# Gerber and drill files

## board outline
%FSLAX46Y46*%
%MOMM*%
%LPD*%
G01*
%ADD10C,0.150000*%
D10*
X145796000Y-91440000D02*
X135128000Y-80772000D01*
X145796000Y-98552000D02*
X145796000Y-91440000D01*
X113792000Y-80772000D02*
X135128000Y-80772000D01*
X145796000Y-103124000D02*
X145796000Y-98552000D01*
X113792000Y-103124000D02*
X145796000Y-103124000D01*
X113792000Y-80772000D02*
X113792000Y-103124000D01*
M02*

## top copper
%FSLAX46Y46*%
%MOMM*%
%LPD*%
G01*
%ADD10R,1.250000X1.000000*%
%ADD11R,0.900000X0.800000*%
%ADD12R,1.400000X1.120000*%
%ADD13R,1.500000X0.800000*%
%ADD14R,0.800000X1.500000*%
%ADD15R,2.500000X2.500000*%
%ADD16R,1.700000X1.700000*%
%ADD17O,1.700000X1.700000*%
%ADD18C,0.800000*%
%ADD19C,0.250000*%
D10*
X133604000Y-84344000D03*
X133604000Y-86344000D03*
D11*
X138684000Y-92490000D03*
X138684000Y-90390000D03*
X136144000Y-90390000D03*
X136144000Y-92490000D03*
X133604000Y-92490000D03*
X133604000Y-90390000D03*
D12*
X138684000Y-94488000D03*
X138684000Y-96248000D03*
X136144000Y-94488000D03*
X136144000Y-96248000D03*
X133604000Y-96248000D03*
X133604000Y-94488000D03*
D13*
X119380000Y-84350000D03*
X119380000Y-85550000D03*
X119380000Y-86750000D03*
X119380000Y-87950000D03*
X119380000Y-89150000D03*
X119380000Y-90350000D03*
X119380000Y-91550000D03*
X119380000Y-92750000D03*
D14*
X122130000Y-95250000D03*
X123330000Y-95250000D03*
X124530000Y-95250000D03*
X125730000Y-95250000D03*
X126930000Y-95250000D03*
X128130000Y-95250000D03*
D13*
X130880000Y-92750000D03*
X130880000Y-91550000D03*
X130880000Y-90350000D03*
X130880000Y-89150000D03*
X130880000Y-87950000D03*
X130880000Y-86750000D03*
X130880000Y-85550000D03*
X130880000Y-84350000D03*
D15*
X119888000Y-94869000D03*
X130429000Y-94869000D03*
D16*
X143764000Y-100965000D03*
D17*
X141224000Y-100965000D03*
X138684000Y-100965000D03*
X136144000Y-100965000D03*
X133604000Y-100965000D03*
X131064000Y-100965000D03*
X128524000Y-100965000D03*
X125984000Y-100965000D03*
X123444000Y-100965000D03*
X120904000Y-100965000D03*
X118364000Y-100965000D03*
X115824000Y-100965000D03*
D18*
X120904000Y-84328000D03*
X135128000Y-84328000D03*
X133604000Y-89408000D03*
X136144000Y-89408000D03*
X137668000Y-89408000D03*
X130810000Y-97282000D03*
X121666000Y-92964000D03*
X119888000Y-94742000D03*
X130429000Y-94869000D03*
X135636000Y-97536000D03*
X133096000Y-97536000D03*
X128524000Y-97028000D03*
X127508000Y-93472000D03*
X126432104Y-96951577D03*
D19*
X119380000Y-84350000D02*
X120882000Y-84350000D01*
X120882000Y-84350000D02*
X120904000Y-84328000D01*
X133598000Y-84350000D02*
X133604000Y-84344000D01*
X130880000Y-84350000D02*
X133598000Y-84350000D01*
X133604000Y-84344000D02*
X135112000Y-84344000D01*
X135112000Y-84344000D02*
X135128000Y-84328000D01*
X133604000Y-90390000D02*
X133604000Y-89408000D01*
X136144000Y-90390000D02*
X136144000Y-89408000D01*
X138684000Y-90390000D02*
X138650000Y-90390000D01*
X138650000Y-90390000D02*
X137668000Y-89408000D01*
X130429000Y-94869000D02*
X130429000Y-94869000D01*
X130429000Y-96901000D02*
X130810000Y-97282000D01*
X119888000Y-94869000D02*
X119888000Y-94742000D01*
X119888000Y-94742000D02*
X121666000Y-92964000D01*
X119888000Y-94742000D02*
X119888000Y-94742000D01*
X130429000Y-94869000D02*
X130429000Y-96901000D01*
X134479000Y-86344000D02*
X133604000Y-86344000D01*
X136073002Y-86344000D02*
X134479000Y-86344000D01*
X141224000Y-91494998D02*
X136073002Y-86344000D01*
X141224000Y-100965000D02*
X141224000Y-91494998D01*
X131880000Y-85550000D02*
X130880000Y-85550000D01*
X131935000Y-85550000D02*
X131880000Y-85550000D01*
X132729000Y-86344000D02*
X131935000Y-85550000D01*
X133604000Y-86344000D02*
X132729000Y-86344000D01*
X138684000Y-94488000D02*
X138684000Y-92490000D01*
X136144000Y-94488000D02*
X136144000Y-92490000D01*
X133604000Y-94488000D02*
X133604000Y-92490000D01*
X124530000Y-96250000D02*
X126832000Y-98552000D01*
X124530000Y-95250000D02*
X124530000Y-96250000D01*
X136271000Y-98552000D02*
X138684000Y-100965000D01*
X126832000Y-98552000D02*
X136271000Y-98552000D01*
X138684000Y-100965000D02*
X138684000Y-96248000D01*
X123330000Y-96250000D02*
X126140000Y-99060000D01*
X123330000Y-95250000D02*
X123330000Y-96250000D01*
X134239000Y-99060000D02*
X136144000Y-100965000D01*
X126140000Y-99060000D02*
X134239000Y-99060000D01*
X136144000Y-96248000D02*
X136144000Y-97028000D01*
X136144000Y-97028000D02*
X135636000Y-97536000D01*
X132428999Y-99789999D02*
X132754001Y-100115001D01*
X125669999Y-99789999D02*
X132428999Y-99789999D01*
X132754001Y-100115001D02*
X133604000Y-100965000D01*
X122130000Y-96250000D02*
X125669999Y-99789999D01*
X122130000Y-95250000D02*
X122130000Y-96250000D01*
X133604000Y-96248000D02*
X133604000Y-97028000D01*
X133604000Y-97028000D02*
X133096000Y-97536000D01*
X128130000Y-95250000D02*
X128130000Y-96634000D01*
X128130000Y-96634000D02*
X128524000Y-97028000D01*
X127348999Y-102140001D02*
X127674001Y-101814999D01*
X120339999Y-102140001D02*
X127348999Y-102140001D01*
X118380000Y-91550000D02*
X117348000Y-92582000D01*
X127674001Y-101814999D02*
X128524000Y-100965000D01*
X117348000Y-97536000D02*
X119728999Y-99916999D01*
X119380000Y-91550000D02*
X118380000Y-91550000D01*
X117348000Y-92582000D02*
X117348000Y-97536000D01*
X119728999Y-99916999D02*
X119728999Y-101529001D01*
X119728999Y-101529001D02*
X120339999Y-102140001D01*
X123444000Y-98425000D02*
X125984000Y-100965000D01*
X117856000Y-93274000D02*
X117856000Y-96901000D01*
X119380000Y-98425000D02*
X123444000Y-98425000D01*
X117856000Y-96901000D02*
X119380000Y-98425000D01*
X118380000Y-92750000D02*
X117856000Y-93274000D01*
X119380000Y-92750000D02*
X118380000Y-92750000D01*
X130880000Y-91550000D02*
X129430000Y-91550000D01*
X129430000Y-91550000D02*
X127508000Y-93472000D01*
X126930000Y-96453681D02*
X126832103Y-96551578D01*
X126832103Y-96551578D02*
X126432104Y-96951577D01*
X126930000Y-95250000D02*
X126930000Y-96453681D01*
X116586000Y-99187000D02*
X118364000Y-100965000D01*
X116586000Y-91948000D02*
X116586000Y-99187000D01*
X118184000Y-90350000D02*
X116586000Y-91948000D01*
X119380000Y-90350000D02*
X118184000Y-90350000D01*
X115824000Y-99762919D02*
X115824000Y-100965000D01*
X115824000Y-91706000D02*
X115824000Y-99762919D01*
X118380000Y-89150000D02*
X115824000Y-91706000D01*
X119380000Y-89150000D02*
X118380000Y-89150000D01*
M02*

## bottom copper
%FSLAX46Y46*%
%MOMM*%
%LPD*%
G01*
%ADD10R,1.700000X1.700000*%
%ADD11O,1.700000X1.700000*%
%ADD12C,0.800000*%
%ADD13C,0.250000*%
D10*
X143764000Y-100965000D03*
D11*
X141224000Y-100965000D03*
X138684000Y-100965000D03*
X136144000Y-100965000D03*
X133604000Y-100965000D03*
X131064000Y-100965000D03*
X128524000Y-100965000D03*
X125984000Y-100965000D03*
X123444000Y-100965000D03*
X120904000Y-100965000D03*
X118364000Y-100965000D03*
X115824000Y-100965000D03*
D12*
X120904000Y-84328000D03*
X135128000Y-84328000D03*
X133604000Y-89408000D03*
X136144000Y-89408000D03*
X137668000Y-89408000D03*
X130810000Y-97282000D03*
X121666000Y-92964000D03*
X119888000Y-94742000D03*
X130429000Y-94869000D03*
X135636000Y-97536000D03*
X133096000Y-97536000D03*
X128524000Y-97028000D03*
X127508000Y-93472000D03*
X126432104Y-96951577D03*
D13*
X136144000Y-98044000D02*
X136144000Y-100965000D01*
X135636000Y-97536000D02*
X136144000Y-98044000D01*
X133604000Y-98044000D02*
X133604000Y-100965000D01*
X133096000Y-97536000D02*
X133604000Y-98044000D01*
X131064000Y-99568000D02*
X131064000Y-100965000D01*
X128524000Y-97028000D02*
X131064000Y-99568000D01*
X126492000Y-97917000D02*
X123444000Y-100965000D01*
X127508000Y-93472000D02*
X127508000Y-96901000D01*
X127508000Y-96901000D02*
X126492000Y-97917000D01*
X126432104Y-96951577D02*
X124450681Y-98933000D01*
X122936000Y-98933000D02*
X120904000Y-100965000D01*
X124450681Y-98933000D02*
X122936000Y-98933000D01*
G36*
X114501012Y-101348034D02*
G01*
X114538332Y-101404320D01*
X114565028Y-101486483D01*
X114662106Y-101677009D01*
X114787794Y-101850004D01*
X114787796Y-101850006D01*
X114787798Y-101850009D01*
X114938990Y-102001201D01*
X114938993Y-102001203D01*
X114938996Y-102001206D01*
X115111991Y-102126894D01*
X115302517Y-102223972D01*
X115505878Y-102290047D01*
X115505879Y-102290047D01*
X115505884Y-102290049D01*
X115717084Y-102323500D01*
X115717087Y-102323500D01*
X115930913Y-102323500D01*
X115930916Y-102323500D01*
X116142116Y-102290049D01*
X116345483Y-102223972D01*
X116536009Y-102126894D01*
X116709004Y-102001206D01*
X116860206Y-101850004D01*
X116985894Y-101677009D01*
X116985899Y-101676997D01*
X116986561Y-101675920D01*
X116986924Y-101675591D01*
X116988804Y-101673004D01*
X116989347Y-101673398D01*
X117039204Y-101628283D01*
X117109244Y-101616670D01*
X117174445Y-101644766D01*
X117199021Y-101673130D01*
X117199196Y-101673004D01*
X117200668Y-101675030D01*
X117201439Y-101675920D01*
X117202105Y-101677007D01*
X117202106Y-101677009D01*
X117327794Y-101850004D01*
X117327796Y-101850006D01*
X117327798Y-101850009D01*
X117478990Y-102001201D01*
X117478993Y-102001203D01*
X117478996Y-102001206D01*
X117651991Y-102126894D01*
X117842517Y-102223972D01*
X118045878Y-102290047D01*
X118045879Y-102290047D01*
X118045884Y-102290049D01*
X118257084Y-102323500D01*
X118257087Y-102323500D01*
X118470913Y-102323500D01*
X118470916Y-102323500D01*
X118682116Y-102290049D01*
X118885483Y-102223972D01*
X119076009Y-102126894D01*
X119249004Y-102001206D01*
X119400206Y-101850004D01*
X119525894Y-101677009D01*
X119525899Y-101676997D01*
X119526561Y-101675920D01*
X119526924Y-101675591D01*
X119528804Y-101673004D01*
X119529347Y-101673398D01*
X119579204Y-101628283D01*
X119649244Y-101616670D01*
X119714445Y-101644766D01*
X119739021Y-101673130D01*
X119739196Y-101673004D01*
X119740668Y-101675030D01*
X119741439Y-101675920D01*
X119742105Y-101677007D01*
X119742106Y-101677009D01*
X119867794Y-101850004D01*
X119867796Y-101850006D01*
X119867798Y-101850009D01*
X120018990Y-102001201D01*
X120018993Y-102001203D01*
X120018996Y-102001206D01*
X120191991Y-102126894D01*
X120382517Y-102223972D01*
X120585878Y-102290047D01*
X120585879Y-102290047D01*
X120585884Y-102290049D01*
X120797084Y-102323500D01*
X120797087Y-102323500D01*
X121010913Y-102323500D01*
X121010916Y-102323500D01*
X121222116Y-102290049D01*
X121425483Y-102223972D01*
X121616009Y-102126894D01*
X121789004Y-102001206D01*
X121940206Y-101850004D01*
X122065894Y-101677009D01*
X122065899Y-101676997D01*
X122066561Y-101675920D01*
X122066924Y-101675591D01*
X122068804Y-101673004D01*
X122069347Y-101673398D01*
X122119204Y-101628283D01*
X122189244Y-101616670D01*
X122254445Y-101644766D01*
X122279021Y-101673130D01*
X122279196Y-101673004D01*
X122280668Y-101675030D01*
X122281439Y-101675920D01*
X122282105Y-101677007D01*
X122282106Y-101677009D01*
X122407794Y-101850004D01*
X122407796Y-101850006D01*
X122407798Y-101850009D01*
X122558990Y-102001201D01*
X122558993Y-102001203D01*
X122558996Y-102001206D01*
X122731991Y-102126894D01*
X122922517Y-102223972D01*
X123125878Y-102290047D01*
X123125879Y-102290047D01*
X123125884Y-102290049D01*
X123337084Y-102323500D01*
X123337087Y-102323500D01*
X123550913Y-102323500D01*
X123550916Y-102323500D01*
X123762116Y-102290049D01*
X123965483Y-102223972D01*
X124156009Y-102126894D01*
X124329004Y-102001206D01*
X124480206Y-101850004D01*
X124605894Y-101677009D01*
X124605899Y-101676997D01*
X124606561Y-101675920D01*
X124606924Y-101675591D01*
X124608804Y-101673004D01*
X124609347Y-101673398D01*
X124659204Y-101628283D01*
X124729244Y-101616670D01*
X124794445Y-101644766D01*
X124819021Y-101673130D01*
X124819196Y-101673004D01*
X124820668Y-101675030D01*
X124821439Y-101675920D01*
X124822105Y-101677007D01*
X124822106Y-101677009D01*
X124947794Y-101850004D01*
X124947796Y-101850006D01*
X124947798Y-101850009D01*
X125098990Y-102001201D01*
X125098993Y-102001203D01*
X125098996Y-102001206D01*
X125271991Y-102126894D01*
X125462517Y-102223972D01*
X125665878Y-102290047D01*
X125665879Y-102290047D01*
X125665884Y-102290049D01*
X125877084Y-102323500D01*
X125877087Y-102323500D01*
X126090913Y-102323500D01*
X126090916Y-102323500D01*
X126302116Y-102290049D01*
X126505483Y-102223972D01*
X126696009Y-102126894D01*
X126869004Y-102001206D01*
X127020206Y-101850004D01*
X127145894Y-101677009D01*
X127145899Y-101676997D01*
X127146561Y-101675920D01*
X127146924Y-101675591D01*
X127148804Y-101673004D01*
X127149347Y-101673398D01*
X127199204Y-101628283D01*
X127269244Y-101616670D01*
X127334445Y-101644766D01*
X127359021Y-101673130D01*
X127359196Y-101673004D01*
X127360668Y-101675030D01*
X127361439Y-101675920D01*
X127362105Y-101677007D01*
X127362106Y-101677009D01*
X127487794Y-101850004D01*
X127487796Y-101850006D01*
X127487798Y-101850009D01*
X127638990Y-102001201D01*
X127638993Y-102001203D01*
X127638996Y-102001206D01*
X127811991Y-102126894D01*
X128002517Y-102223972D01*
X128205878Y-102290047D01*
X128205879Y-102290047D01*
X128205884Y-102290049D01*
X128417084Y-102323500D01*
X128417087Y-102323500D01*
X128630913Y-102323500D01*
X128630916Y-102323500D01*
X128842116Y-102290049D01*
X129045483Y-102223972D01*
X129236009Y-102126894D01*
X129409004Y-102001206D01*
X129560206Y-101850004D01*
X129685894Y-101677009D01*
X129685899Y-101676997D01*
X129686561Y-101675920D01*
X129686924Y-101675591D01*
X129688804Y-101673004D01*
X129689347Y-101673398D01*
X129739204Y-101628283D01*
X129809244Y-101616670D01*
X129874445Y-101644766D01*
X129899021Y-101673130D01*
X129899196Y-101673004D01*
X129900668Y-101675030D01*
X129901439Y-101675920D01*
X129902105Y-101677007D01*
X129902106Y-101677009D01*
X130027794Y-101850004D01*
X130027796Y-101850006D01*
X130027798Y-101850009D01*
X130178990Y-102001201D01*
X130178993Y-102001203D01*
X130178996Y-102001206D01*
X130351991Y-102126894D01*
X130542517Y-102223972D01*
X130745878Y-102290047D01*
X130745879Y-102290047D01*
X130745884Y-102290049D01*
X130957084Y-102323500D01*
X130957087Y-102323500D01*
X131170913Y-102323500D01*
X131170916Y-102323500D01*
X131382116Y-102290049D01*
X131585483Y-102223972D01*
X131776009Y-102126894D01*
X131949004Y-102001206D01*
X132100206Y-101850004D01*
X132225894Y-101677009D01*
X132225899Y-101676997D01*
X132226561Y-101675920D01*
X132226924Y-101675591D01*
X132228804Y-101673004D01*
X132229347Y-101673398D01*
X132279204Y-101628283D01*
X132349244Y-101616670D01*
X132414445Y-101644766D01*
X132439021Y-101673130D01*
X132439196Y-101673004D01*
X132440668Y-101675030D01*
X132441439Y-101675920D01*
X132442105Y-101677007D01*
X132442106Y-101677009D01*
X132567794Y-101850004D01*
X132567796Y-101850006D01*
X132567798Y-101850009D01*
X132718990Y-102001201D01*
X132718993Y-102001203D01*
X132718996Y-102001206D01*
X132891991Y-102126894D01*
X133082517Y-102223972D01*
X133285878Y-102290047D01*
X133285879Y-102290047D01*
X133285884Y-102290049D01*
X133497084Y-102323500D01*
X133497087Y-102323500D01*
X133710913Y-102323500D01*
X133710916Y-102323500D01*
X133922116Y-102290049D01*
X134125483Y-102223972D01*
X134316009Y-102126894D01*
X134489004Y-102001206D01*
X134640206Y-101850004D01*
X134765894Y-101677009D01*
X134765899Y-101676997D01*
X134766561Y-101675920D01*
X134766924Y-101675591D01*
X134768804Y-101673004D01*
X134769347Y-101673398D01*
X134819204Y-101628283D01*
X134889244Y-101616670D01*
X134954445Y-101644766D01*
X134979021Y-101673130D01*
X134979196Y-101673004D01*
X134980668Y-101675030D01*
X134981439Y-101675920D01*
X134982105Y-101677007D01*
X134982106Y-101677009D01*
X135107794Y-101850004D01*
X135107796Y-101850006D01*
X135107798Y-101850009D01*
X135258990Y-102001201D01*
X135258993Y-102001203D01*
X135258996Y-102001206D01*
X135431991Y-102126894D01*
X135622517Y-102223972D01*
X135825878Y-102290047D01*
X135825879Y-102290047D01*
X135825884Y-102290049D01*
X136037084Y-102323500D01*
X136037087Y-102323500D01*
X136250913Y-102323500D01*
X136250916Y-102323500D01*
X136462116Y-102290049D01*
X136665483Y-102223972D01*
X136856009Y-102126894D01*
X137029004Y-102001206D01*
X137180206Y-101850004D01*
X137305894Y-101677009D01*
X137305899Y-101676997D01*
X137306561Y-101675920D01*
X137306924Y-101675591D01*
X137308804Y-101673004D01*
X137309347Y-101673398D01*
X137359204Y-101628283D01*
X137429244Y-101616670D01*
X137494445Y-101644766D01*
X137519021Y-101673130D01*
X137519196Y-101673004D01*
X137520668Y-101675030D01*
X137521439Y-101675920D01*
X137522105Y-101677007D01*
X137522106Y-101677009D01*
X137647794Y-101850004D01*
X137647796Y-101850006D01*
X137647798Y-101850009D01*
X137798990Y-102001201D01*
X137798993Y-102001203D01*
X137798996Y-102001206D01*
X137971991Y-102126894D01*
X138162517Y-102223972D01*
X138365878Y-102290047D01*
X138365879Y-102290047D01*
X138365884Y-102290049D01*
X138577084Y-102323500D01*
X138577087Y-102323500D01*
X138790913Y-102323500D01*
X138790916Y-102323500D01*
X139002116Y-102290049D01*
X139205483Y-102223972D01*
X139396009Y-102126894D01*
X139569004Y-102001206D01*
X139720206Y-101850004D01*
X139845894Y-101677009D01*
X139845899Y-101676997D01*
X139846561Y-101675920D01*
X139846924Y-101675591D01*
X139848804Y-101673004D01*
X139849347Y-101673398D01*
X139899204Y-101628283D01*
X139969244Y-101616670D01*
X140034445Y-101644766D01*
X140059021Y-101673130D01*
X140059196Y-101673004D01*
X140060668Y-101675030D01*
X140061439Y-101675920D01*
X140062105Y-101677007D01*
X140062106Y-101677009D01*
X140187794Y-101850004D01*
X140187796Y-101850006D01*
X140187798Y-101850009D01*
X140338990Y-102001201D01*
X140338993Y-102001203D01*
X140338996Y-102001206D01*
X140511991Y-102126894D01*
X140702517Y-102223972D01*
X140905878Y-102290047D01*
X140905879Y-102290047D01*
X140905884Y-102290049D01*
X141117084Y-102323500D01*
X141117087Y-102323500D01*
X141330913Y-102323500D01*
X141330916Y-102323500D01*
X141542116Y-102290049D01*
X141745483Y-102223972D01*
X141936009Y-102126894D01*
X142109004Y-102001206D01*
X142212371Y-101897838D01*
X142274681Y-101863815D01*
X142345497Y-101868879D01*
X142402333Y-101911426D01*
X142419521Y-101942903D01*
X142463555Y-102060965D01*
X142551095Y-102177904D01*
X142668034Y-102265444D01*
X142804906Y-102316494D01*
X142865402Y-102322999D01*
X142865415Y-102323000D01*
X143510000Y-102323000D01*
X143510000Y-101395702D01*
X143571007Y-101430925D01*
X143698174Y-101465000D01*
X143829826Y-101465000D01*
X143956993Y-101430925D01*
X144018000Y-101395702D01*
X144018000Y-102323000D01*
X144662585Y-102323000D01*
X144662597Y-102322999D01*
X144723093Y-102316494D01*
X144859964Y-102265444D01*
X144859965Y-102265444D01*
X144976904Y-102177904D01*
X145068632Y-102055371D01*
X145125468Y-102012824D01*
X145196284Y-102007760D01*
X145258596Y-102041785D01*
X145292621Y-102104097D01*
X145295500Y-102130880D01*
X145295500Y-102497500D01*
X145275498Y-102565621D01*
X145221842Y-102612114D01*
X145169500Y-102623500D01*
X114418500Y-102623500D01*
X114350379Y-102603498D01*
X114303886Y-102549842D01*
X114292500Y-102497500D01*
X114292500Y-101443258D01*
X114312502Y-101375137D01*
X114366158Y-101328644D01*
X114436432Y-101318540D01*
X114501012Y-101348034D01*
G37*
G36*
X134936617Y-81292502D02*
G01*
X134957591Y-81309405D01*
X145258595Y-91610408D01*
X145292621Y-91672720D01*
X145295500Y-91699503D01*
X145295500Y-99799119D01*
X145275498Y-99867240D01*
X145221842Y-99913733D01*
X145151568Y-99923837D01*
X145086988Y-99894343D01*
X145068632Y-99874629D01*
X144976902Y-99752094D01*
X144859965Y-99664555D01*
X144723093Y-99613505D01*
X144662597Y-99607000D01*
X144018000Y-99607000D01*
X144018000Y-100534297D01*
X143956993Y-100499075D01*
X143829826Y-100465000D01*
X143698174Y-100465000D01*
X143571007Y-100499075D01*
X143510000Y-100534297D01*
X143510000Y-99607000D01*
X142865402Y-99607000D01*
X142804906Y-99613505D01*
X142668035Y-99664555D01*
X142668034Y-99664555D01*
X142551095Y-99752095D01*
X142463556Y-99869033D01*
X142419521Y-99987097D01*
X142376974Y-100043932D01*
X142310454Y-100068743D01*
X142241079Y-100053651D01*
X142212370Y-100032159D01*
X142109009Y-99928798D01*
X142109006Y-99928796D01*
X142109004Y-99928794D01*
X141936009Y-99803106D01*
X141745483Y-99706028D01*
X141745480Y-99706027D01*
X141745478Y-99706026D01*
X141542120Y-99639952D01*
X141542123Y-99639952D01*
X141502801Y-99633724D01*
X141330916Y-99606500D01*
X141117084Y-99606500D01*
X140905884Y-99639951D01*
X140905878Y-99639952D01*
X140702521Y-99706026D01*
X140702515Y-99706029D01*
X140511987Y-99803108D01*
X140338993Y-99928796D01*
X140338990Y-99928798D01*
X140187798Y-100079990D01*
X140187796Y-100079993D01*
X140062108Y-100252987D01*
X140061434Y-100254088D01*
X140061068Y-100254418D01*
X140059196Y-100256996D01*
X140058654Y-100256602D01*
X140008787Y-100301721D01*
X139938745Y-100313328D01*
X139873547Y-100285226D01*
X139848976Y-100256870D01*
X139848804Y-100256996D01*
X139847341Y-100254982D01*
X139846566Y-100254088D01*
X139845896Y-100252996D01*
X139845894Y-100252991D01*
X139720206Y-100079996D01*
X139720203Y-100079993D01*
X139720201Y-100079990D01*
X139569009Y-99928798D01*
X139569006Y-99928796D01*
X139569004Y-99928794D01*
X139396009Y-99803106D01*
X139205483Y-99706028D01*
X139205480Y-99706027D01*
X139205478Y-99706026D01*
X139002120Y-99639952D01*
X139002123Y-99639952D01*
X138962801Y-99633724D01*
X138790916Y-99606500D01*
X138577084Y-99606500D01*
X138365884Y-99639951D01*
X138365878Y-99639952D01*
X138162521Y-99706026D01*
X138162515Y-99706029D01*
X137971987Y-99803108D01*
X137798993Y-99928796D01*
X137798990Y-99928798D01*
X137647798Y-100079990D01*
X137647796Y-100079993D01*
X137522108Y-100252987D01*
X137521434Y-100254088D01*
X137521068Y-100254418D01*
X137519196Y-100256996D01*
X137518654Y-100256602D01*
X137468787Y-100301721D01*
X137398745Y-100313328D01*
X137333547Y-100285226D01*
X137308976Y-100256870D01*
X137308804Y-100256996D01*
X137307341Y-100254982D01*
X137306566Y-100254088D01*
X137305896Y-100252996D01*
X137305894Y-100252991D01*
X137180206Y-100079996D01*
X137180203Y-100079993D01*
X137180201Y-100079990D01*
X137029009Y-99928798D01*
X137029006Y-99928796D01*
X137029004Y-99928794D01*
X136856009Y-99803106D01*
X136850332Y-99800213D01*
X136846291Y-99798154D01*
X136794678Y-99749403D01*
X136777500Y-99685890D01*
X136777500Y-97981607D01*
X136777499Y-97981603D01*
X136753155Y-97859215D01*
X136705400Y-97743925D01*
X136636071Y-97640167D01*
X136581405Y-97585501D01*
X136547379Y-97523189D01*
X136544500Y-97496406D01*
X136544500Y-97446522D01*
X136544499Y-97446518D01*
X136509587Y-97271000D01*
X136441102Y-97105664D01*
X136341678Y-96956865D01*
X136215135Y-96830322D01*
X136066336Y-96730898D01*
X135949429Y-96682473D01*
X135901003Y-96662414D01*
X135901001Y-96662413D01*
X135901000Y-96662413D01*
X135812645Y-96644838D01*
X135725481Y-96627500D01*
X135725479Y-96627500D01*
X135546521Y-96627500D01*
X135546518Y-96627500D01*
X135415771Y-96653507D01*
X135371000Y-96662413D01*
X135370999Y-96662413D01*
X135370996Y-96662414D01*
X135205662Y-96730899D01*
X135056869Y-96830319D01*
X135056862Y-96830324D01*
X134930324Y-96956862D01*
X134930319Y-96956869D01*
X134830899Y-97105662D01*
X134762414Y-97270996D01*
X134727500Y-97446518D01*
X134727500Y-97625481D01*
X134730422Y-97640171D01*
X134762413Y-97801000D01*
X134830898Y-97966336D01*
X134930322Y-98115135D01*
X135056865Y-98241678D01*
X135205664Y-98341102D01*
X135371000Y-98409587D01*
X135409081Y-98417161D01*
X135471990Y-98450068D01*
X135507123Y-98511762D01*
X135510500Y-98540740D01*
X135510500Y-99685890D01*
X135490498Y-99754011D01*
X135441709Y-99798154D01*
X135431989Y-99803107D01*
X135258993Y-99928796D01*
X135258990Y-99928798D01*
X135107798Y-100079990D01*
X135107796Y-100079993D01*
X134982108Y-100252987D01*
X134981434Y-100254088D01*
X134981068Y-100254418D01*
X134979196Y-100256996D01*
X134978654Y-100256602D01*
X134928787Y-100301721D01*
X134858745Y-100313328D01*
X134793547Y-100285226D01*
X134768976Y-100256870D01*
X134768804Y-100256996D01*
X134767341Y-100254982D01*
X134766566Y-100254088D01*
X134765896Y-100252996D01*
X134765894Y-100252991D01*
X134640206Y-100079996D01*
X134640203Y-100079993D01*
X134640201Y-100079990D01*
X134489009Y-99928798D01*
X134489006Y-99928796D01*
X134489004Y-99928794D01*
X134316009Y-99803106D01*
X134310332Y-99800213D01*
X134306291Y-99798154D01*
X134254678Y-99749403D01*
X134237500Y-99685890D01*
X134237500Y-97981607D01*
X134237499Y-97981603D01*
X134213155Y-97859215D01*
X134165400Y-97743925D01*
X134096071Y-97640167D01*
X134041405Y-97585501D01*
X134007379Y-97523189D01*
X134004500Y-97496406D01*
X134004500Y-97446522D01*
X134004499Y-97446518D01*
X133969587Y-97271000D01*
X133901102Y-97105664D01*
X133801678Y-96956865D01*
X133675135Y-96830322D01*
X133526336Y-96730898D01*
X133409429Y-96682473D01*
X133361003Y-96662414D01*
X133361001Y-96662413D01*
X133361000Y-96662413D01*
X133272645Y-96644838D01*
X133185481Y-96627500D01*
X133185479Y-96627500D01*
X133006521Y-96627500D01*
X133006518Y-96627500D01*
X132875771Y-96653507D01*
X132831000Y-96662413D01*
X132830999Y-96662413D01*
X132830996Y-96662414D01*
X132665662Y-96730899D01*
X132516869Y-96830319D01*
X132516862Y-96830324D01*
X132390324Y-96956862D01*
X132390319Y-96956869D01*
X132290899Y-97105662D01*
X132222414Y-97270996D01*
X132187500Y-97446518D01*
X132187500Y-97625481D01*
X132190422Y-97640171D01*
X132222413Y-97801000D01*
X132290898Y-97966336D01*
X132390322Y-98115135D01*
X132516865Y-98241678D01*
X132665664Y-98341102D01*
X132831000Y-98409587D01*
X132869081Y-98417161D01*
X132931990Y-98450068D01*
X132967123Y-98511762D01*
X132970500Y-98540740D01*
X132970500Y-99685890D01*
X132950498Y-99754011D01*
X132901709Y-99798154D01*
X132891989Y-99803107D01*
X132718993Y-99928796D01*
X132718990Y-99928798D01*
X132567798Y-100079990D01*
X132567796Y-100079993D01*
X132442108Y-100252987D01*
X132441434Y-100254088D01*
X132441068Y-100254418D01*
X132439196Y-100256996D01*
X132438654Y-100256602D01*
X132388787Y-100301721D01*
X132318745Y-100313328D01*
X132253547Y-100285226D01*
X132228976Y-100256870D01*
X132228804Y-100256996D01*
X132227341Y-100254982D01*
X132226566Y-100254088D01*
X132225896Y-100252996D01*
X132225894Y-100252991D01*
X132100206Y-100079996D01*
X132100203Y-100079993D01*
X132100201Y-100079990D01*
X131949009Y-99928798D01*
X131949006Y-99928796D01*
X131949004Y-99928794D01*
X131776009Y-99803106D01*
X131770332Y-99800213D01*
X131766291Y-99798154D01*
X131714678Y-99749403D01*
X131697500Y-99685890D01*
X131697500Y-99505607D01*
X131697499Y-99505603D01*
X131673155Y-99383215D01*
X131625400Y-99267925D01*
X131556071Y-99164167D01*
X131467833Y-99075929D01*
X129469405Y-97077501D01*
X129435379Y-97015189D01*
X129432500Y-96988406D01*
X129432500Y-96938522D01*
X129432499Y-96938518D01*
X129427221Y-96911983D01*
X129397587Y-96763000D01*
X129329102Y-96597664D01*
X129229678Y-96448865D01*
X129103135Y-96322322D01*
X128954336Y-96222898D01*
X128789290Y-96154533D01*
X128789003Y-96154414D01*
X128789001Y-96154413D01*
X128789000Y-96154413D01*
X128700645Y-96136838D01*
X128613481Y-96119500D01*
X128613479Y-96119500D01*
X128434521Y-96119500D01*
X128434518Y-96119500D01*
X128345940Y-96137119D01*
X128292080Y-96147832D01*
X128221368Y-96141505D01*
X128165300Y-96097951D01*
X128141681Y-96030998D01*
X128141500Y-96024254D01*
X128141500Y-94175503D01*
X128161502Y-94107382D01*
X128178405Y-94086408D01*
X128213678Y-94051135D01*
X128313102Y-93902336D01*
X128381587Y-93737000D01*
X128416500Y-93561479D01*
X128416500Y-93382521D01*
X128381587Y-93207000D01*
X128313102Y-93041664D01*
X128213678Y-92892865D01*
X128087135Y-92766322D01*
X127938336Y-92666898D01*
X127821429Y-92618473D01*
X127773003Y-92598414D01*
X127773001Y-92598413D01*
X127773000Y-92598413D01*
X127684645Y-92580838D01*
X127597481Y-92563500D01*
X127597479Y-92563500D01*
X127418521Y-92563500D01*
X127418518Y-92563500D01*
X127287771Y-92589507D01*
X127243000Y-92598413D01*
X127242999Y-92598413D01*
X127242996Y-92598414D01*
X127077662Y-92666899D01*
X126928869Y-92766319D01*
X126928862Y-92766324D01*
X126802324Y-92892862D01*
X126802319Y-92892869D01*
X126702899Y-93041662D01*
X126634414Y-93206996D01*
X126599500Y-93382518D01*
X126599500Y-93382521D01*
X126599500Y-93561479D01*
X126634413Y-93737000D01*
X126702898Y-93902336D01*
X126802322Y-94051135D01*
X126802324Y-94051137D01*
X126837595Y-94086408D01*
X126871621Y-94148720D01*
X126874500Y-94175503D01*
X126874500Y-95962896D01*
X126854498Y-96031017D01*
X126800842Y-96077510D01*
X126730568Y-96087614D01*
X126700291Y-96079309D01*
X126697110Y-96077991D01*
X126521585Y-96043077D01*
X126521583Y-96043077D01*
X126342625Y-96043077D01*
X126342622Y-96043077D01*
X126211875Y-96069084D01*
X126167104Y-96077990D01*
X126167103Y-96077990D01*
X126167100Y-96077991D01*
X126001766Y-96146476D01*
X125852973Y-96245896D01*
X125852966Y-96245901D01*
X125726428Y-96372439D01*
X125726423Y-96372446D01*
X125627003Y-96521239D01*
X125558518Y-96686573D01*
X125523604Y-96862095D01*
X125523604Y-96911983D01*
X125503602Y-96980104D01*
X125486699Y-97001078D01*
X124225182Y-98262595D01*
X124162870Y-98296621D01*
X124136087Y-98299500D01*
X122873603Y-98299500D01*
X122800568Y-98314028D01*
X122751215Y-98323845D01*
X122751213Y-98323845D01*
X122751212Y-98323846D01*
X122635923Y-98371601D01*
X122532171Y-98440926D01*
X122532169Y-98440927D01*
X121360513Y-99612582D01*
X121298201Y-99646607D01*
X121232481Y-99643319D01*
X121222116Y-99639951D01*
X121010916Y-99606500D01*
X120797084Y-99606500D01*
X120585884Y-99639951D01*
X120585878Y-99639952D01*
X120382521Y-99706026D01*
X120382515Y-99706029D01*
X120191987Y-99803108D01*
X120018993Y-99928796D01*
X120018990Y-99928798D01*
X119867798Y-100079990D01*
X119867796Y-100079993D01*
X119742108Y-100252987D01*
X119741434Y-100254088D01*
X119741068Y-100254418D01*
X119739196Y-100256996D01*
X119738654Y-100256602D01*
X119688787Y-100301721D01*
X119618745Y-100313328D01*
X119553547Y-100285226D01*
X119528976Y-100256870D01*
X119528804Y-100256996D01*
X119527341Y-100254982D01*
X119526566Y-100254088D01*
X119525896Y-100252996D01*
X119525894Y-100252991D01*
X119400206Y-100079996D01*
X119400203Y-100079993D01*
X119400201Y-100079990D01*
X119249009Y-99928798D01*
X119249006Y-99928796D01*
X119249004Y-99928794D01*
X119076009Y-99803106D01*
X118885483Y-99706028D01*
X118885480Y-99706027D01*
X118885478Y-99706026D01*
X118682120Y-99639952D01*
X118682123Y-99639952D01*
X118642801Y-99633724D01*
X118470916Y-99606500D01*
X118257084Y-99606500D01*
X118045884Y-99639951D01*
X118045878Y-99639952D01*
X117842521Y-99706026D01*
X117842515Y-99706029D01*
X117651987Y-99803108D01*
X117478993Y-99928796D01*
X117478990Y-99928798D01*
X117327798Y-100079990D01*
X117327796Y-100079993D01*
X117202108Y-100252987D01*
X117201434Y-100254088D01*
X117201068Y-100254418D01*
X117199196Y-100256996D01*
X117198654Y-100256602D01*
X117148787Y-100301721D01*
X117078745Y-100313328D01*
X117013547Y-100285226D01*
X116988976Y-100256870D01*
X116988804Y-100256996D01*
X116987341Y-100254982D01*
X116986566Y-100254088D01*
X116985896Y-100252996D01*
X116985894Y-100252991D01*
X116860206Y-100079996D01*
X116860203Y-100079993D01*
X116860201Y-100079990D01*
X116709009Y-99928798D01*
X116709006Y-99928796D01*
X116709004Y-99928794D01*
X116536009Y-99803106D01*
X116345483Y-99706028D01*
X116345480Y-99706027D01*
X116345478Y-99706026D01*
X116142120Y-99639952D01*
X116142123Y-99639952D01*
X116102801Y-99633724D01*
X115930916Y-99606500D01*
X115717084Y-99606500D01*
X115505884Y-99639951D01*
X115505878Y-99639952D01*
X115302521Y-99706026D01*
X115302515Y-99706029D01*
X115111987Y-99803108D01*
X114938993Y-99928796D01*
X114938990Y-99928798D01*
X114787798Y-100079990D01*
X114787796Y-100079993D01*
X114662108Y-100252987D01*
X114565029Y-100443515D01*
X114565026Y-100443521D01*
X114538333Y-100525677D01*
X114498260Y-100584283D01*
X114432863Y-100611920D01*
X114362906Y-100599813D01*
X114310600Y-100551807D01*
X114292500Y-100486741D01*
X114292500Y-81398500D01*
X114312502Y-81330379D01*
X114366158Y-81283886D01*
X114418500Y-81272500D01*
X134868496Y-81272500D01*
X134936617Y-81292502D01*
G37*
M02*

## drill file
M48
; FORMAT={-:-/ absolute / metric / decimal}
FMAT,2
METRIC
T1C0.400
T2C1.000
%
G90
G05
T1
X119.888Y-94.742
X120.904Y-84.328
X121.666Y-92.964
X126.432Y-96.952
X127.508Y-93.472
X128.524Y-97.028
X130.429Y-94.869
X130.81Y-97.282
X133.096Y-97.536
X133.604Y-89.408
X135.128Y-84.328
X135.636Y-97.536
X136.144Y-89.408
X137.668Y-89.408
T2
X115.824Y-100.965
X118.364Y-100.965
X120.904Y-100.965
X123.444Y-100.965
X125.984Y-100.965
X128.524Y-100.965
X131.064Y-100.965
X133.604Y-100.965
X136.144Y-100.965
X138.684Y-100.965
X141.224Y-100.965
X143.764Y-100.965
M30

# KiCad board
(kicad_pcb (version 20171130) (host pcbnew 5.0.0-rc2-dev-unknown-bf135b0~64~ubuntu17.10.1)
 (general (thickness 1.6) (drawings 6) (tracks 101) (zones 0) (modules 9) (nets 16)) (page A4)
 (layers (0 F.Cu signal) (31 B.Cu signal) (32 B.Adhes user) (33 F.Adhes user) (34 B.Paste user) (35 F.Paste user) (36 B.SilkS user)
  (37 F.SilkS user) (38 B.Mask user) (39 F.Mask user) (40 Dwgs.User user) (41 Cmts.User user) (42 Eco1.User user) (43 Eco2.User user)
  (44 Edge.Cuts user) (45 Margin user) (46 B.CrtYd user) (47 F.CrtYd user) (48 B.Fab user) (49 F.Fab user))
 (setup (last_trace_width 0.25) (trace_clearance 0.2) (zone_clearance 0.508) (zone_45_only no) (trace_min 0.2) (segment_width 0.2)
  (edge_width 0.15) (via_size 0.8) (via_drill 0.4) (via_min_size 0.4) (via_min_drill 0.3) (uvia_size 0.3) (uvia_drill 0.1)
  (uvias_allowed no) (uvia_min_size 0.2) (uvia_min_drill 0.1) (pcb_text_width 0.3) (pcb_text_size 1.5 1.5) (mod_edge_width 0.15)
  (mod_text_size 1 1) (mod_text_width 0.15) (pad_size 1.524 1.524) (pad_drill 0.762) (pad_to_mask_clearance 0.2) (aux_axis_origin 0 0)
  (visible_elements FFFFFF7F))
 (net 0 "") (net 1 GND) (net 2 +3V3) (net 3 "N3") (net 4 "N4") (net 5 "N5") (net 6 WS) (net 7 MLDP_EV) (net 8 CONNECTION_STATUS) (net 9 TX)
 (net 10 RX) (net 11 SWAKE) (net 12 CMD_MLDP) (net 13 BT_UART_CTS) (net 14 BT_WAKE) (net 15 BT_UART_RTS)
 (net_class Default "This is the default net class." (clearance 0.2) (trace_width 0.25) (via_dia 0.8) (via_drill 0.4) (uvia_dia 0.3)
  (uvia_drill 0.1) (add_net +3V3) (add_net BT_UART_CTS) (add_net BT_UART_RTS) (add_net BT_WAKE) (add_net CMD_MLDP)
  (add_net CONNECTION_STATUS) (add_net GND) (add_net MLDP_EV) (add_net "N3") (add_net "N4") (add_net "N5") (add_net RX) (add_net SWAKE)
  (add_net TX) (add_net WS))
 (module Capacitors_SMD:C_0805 (layer F.Cu) (at 133.604 85.344 90)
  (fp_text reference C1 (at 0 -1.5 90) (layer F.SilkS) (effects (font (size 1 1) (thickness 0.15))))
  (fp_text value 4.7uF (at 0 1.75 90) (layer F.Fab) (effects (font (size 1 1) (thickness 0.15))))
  (pad 2 smd rect (at 1 0 90) (size 1 1.25) (layers F.Cu F.Paste F.Mask) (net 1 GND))
  (pad 1 smd rect (at -1 0 90) (size 1 1.25) (layers F.Cu F.Paste F.Mask) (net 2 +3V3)))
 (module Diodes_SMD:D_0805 (layer F.Cu) (at 138.684 91.44 270)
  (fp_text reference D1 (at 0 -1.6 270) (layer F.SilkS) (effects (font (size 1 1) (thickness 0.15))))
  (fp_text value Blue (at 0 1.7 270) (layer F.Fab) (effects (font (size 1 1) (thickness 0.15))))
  (pad 2 smd rect (at 1.05 0 270) (size 0.8 0.9) (layers F.Cu F.Paste F.Mask) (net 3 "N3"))
  (pad 1 smd rect (at -1.05 0 270) (size 0.8 0.9) (layers F.Cu F.Paste F.Mask) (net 1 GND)))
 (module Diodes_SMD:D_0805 (layer F.Cu) (at 136.144 91.44 270)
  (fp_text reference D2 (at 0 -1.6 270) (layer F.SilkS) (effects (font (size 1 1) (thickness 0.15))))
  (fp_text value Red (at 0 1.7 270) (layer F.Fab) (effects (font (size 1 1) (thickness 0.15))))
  (pad 1 smd rect (at -1.05 0 270) (size 0.8 0.9) (layers F.Cu F.Paste F.Mask) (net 1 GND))
  (pad 2 smd rect (at 1.05 0 270) (size 0.8 0.9) (layers F.Cu F.Paste F.Mask) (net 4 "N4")))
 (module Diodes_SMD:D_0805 (layer F.Cu) (at 133.604 91.44 270)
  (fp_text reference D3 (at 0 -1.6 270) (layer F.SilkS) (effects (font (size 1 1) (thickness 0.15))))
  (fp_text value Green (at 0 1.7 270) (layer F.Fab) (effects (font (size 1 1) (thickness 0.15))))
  (pad 2 smd rect (at 1.05 0 270) (size 0.8 0.9) (layers F.Cu F.Paste F.Mask) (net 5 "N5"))
  (pad 1 smd rect (at -1.05 0 270) (size 0.8 0.9) (layers F.Cu F.Paste F.Mask) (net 1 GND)))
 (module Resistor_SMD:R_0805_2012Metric (layer F.Cu) (at 138.684 95.368 270)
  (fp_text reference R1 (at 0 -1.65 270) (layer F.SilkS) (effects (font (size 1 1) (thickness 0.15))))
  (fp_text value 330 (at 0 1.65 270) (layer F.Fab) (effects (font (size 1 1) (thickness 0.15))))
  (pad 1 smd rect (at -0.88 0 270) (size 1.12 1.4) (layers F.Cu F.Paste F.Mask) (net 3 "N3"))
  (pad 2 smd rect (at 0.88 0 270) (size 1.12 1.4) (layers F.Cu F.Paste F.Mask) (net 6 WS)))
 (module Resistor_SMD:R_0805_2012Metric (layer F.Cu) (at 136.144 95.368 90)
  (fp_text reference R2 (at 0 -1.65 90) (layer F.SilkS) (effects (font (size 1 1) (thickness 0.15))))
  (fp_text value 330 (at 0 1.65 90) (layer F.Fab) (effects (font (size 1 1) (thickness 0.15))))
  (pad 2 smd rect (at 0.88 0 90) (size 1.12 1.4) (layers F.Cu F.Paste F.Mask) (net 4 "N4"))
  (pad 1 smd rect (at -0.88 0 90) (size 1.12 1.4) (layers F.Cu F.Paste F.Mask) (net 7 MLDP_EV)))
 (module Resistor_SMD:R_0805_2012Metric (layer F.Cu) (at 133.604 95.368 90)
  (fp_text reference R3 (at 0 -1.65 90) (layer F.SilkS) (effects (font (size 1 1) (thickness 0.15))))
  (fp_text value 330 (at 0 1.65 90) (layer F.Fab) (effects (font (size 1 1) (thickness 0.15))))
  (pad 1 smd rect (at -0.88 0 90) (size 1.12 1.4) (layers F.Cu F.Paste F.Mask) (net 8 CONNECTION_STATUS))
  (pad 2 smd rect (at 0.88 0 90) (size 1.12 1.4) (layers F.Cu F.Paste F.Mask) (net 5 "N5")))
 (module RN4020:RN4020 (layer F.Cu) (at 119.38 95.25)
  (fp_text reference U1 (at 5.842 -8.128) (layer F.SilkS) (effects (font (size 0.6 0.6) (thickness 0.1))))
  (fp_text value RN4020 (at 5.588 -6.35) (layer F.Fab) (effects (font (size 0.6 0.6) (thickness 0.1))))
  (pad 1 smd rect (at 0 -10.9) (size 1.5 0.8) (layers F.Cu F.Paste F.Mask) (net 1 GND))
  (pad 2 smd rect (at 0 -9.7) (size 1.5 0.8) (layers F.Cu F.Paste F.Mask))
  (pad 3 smd rect (at 0 -8.5) (size 1.5 0.8) (layers F.Cu F.Paste F.Mask))
  (pad 4 smd rect (at 0 -7.3) (size 1.5 0.8) (layers F.Cu F.Paste F.Mask))
  (pad 5 smd rect (at 0 -6.1) (size 1.5 0.8) (layers F.Cu F.Paste F.Mask) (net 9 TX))
  (pad 6 smd rect (at 0 -4.9) (size 1.5 0.8) (layers F.Cu F.Paste F.Mask) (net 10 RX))
  (pad 7 smd rect (at 0 -3.7) (size 1.5 0.8) (layers F.Cu F.Paste F.Mask) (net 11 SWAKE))
  (pad 8 smd rect (at 0 -2.5) (size 1.5 0.8) (layers F.Cu F.Paste F.Mask) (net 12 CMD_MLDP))
  (pad 10 smd rect (at 2.75 0) (size 0.8 1.5) (layers F.Cu F.Paste F.Mask) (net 8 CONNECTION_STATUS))
  (pad 11 smd rect (at 3.95 0) (size 0.8 1.5) (layers F.Cu F.Paste F.Mask) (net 7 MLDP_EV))
  (pad 12 smd rect (at 5.15 0) (size 0.8 1.5) (layers F.Cu F.Paste F.Mask) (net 6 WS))
  (pad 13 smd rect (at 6.35 0) (size 0.8 1.5) (layers F.Cu F.Paste F.Mask))
  (pad 14 smd rect (at 7.55 0) (size 0.8 1.5) (layers F.Cu F.Paste F.Mask) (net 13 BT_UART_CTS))
  (pad 15 smd rect (at 8.75 0) (size 0.8 1.5) (layers F.Cu F.Paste F.Mask) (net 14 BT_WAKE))
  (pad 17 smd rect (at 11.5 -2.5) (size 1.5 0.8) (layers F.Cu F.Paste F.Mask))
  (pad 18 smd rect (at 11.5 -3.7) (size 1.5 0.8) (layers F.Cu F.Paste F.Mask) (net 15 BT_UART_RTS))
  (pad 19 smd rect (at 11.5 -4.9) (size 1.5 0.8) (layers F.Cu F.Paste F.Mask))
  (pad 20 smd rect (at 11.5 -6.1) (size 1.5 0.8) (layers F.Cu F.Paste F.Mask))
  (pad 21 smd rect (at 11.5 -7.3) (size 1.5 0.8) (layers F.Cu F.Paste F.Mask))
  (pad 22 smd rect (at 11.5 -8.5) (size 1.5 0.8) (layers F.Cu F.Paste F.Mask))
  (pad 23 smd rect (at 11.5 -9.7) (size 1.5 0.8) (layers F.Cu F.Paste F.Mask) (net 2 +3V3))
  (pad 24 smd rect (at 11.5 -10.9) (size 1.5 0.8) (layers F.Cu F.Paste F.Mask) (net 1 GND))
  (pad 9 smd rect (at 0.508 -0.381) (size 2.5 2.5) (layers F.Cu F.Paste F.Mask) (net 1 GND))
  (pad 16 smd rect (at 11.049 -0.381) (size 2.5 2.5) (layers F.Cu F.Paste F.Mask) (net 1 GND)))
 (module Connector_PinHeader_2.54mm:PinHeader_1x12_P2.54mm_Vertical (layer F.Cu) (at 143.764 100.965 270)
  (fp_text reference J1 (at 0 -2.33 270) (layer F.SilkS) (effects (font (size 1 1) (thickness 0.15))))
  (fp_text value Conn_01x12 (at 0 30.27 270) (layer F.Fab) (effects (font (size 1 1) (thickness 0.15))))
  (pad 1 thru_hole rect (at 0 0 270) (size 1.7 1.7) (drill 1) (layers *.Cu *.Mask) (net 1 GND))
  (pad 2 thru_hole oval (at 0 2.54 270) (size 1.7 1.7) (drill 1) (layers *.Cu *.Mask) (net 2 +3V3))
  (pad 3 thru_hole oval (at 0 5.08 270) (size 1.7 1.7) (drill 1) (layers *.Cu *.Mask) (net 6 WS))
  (pad 4 thru_hole oval (at 0 7.62 270) (size 1.7 1.7) (drill 1) (layers *.Cu *.Mask) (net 7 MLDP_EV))
  (pad 5 thru_hole oval (at 0 10.16 270) (size 1.7 1.7) (drill 1) (layers *.Cu *.Mask) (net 8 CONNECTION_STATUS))
  (pad 6 thru_hole oval (at 0 12.7 270) (size 1.7 1.7) (drill 1) (layers *.Cu *.Mask) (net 14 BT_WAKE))
  (pad 7 thru_hole oval (at 0 15.24 270) (size 1.7 1.7) (drill 1) (layers *.Cu *.Mask) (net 11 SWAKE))
  (pad 8 thru_hole oval (at 0 17.78 270) (size 1.7 1.7) (drill 1) (layers *.Cu *.Mask) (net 12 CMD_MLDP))
  (pad 9 thru_hole oval (at 0 20.32 270) (size 1.7 1.7) (drill 1) (layers *.Cu *.Mask) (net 15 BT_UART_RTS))
  (pad 10 thru_hole oval (at 0 22.86 270) (size 1.7 1.7) (drill 1) (layers *.Cu *.Mask) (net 13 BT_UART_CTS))
  (pad 11 thru_hole oval (at 0 25.4 270) (size 1.7 1.7) (drill 1) (layers *.Cu *.Mask) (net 10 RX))
  (pad 12 thru_hole oval (at 0 27.94 270) (size 1.7 1.7) (drill 1) (layers *.Cu *.Mask) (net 9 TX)))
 (gr_line (start 145.796 91.44) (end 135.128 80.772) (layer Edge.Cuts) (width 0.15))
 (gr_line (start 145.796 98.552) (end 145.796 91.44) (layer Edge.Cuts) (width 0.15))
 (gr_line (start 113.792 80.772) (end 135.128 80.772) (layer Edge.Cuts) (width 0.15))
 (gr_line (start 145.796 103.124) (end 145.796 98.552) (layer Edge.Cuts) (width 0.15))
 (gr_line (start 113.792 103.124) (end 145.796 103.124) (layer Edge.Cuts) (width 0.15))
 (gr_line (start 113.792 80.772) (end 113.792 103.124) (layer Edge.Cuts) (width 0.15))
 (via (at 120.904 84.328) (size 0.8) (drill 0.4) (layers F.Cu B.Cu) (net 1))
 (segment (start 119.38 84.35) (end 120.882 84.35) (width 0.25) (layer F.Cu) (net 1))
 (segment (start 120.882 84.35) (end 120.904 84.328) (width 0.25) (layer F.Cu) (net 1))
 (segment (start 133.598 84.35) (end 133.604 84.344) (width 0.25) (layer F.Cu) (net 1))
 (segment (start 130.88 84.35) (end 133.598 84.35) (width 0.25) (layer F.Cu) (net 1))
 (via (at 135.128 84.328) (size 0.8) (drill 0.4) (layers F.Cu B.Cu) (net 1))
 (segment (start 133.604 84.344) (end 135.112 84.344) (width 0.25) (layer F.Cu) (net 1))
 (segment (start 135.112 84.344) (end 135.128 84.328) (width 0.25) (layer F.Cu) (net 1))
 (via (at 133.604 89.408) (size 0.8) (drill 0.4) (layers F.Cu B.Cu) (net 1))
 (segment (start 133.604 90.39) (end 133.604 89.408) (width 0.25) (layer F.Cu) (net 1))
 (via (at 136.144 89.408) (size 0.8) (drill 0.4) (layers F.Cu B.Cu) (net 1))
 (segment (start 136.144 90.39) (end 136.144 89.408) (width 0.25) (layer F.Cu) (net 1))
 (via (at 137.668 89.408) (size 0.8) (drill 0.4) (layers F.Cu B.Cu) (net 1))
 (segment (start 138.684 90.39) (end 138.65 90.39) (width 0.25) (layer F.Cu) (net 1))
 (segment (start 138.65 90.39) (end 137.668 89.408) (width 0.25) (layer F.Cu) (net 1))
 (via (at 130.81 97.282) (size 0.8) (drill 0.4) (layers F.Cu B.Cu) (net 1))
 (segment (start 130.429 94.869) (end 130.429 94.869) (width 0.25) (layer F.Cu) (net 1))
 (segment (start 130.429 96.901) (end 130.81 97.282) (width 0.25) (layer F.Cu) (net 1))
 (via (at 121.666 92.964) (size 0.8) (drill 0.4) (layers F.Cu B.Cu) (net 1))
 (segment (start 119.888 94.869) (end 119.888 94.742) (width 0.25) (layer F.Cu) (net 1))
 (segment (start 119.888 94.742) (end 121.666 92.964) (width 0.25) (layer F.Cu) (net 1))
 (segment (start 119.888 94.742) (end 119.888 94.742) (width 0.25) (layer F.Cu) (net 1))
 (via (at 119.888 94.742) (size 0.8) (drill 0.4) (layers F.Cu B.Cu) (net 1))
 (segment (start 130.429 94.869) (end 130.429 96.901) (width 0.25) (layer F.Cu) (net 1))
 (via (at 130.429 94.869) (size 0.8) (drill 0.4) (layers F.Cu B.Cu) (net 1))
 (segment (start 134.479 86.344) (end 133.604 86.344) (width 0.25) (layer F.Cu) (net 2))
 (segment (start 136.073002 86.344) (end 134.479 86.344) (width 0.25) (layer F.Cu) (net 2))
 (segment (start 141.224 91.494998) (end 136.073002 86.344) (width 0.25) (layer F.Cu) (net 2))
 (segment (start 141.224 100.965) (end 141.224 91.494998) (width 0.25) (layer F.Cu) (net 2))
 (segment (start 131.88 85.55) (end 130.88 85.55) (width 0.25) (layer F.Cu) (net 2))
 (segment (start 131.935 85.55) (end 131.88 85.55) (width 0.25) (layer F.Cu) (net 2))
 (segment (start 132.729 86.344) (end 131.935 85.55) (width 0.25) (layer F.Cu) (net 2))
 (segment (start 133.604 86.344) (end 132.729 86.344) (width 0.25) (layer F.Cu) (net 2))
 (segment (start 138.684 94.488) (end 138.684 92.49) (width 0.25) (layer F.Cu) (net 3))
 (segment (start 136.144 94.488) (end 136.144 92.49) (width 0.25) (layer F.Cu) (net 4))
 (segment (start 133.604 94.488) (end 133.604 92.49) (width 0.25) (layer F.Cu) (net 5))
 (segment (start 124.53 96.25) (end 126.832 98.552) (width 0.25) (layer F.Cu) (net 6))
 (segment (start 124.53 95.25) (end 124.53 96.25) (width 0.25) (layer F.Cu) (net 6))
 (segment (start 136.271 98.552) (end 138.684 100.965) (width 0.25) (layer F.Cu) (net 6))
 (segment (start 126.832 98.552) (end 136.271 98.552) (width 0.25) (layer F.Cu) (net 6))
 (segment (start 138.684 100.965) (end 138.684 96.248) (width 0.25) (layer F.Cu) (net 6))
 (segment (start 123.33 96.25) (end 126.14 99.06) (width 0.25) (layer F.Cu) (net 7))
 (segment (start 123.33 95.25) (end 123.33 96.25) (width 0.25) (layer F.Cu) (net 7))
 (segment (start 134.239 99.06) (end 136.144 100.965) (width 0.25) (layer F.Cu) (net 7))
 (segment (start 126.14 99.06) (end 134.239 99.06) (width 0.25) (layer F.Cu) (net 7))
 (via (at 135.636 97.536) (size 0.8) (drill 0.4) (layers F.Cu B.Cu) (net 7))
 (segment (start 136.144 96.248) (end 136.144 97.028) (width 0.25) (layer F.Cu) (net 7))
 (segment (start 136.144 97.028) (end 135.636 97.536) (width 0.25) (layer F.Cu) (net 7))
 (segment (start 136.144 98.044) (end 136.144 100.965) (width 0.25) (layer B.Cu) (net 7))
 (segment (start 135.636 97.536) (end 136.144 98.044) (width 0.25) (layer B.Cu) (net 7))
 (segment (start 132.428999 99.789999) (end 132.754001 100.115001) (width 0.25) (layer F.Cu) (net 8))
 (segment (start 125.669999 99.789999) (end 132.428999 99.789999) (width 0.25) (layer F.Cu) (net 8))
 (segment (start 132.754001 100.115001) (end 133.604 100.965) (width 0.25) (layer F.Cu) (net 8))
 (segment (start 122.13 96.25) (end 125.669999 99.789999) (width 0.25) (layer F.Cu) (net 8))
 (segment (start 122.13 95.25) (end 122.13 96.25) (width 0.25) (layer F.Cu) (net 8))
 (via (at 133.096 97.536) (size 0.8) (drill 0.4) (layers F.Cu B.Cu) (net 8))
 (segment (start 133.604 96.248) (end 133.604 97.028) (width 0.25) (layer F.Cu) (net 8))
 (segment (start 133.604 97.028) (end 133.096 97.536) (width 0.25) (layer F.Cu) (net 8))
 (segment (start 133.604 98.044) (end 133.604 100.965) (width 0.25) (layer B.Cu) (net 8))
 (segment (start 133.096 97.536) (end 133.604 98.044) (width 0.25) (layer B.Cu) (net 8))
 (segment (start 128.13 95.25) (end 128.13 96.634) (width 0.25) (layer F.Cu) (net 14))
 (via (at 128.524 97.028) (size 0.8) (drill 0.4) (layers F.Cu B.Cu) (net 14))
 (segment (start 128.13 96.634) (end 128.524 97.028) (width 0.25) (layer F.Cu) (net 14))
 (segment (start 131.064 99.568) (end 131.064 100.965) (width 0.25) (layer B.Cu) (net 14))
 (segment (start 128.524 97.028) (end 131.064 99.568) (width 0.25) (layer B.Cu) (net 14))
 (segment (start 127.348999 102.140001) (end 127.674001 101.814999) (width 0.25) (layer F.Cu) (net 11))
 (segment (start 120.339999 102.140001) (end 127.348999 102.140001) (width 0.25) (layer F.Cu) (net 11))
 (segment (start 118.38 91.55) (end 117.348 92.582) (width 0.25) (layer F.Cu) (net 11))
 (segment (start 127.674001 101.814999) (end 128.524 100.965) (width 0.25) (layer F.Cu) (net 11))
 (segment (start 117.348 97.536) (end 119.728999 99.916999) (width 0.25) (layer F.Cu) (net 11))
 (segment (start 119.38 91.55) (end 118.38 91.55) (width 0.25) (layer F.Cu) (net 11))
 (segment (start 117.348 92.582) (end 117.348 97.536) (width 0.25) (layer F.Cu) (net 11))
 (segment (start 119.728999 99.916999) (end 119.728999 101.529001) (width 0.25) (layer F.Cu) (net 11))
 (segment (start 119.728999 101.529001) (end 120.339999 102.140001) (width 0.25) (layer F.Cu) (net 11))
 (segment (start 123.444 98.425) (end 125.984 100.965) (width 0.25) (layer F.Cu) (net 12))
 (segment (start 117.856 93.274) (end 117.856 96.901) (width 0.25) (layer F.Cu) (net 12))
 (segment (start 119.38 98.425) (end 123.444 98.425) (width 0.25) (layer F.Cu) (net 12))
 (segment (start 117.856 96.901) (end 119.38 98.425) (width 0.25) (layer F.Cu) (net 12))
 (segment (start 118.38 92.75) (end 117.856 93.274) (width 0.25) (layer F.Cu) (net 12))
 (segment (start 119.38 92.75) (end 118.38 92.75) (width 0.25) (layer F.Cu) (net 12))
 (via (at 127.508 93.472) (size 0.8) (drill 0.4) (layers F.Cu B.Cu) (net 15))
 (segment (start 130.88 91.55) (end 129.43 91.55) (width 0.25) (layer F.Cu) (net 15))
 (segment (start 129.43 91.55) (end 127.508 93.472) (width 0.25) (layer F.Cu) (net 15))
 (segment (start 126.492 97.917) (end 123.444 100.965) (width 0.25) (layer B.Cu) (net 15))
 (segment (start 127.508 93.472) (end 127.508 96.901) (width 0.25) (layer B.Cu) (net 15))
 (segment (start 127.508 96.901) (end 126.492 97.917) (width 0.25) (layer B.Cu) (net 15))
 (via (at 126.432104 96.951577) (size 0.8) (drill 0.4) (layers F.Cu B.Cu) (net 13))
 (segment (start 126.93 96.453681) (end 126.832103 96.551578) (width 0.25) (layer F.Cu) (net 13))
 (segment (start 126.832103 96.551578) (end 126.432104 96.951577) (width 0.25) (layer F.Cu) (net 13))
 (segment (start 126.93 95.25) (end 126.93 96.453681) (width 0.25) (layer F.Cu) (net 13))
 (segment (start 126.432104 96.951577) (end 124.450681 98.933) (width 0.25) (layer B.Cu) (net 13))
 (segment (start 122.936 98.933) (end 120.904 100.965) (width 0.25) (layer B.Cu) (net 13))
 (segment (start 124.450681 98.933) (end 122.936 98.933) (width 0.25) (layer B.Cu) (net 13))
 (segment (start 116.586 99.187) (end 118.364 100.965) (width 0.25) (layer F.Cu) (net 10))
 (segment (start 116.586 91.948) (end 116.586 99.187) (width 0.25) (layer F.Cu) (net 10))
 (segment (start 118.184 90.35) (end 116.586 91.948) (width 0.25) (layer F.Cu) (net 10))
 (segment (start 119.38 90.35) (end 118.184 90.35) (width 0.25) (layer F.Cu) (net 10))
 (segment (start 115.824 99.762919) (end 115.824 100.965) (width 0.25) (layer F.Cu) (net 9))
 (segment (start 115.824 91.706) (end 115.824 99.762919) (width 0.25) (layer F.Cu) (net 9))
 (segment (start 118.38 89.15) (end 115.824 91.706) (width 0.25) (layer F.Cu) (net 9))
 (segment (start 119.38 89.15) (end 118.38 89.15) (width 0.25) (layer F.Cu) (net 9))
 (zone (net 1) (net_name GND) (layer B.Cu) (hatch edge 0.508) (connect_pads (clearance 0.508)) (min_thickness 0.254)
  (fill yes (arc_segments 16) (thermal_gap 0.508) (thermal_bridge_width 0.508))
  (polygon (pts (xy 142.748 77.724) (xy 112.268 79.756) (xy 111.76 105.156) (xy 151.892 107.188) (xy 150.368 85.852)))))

